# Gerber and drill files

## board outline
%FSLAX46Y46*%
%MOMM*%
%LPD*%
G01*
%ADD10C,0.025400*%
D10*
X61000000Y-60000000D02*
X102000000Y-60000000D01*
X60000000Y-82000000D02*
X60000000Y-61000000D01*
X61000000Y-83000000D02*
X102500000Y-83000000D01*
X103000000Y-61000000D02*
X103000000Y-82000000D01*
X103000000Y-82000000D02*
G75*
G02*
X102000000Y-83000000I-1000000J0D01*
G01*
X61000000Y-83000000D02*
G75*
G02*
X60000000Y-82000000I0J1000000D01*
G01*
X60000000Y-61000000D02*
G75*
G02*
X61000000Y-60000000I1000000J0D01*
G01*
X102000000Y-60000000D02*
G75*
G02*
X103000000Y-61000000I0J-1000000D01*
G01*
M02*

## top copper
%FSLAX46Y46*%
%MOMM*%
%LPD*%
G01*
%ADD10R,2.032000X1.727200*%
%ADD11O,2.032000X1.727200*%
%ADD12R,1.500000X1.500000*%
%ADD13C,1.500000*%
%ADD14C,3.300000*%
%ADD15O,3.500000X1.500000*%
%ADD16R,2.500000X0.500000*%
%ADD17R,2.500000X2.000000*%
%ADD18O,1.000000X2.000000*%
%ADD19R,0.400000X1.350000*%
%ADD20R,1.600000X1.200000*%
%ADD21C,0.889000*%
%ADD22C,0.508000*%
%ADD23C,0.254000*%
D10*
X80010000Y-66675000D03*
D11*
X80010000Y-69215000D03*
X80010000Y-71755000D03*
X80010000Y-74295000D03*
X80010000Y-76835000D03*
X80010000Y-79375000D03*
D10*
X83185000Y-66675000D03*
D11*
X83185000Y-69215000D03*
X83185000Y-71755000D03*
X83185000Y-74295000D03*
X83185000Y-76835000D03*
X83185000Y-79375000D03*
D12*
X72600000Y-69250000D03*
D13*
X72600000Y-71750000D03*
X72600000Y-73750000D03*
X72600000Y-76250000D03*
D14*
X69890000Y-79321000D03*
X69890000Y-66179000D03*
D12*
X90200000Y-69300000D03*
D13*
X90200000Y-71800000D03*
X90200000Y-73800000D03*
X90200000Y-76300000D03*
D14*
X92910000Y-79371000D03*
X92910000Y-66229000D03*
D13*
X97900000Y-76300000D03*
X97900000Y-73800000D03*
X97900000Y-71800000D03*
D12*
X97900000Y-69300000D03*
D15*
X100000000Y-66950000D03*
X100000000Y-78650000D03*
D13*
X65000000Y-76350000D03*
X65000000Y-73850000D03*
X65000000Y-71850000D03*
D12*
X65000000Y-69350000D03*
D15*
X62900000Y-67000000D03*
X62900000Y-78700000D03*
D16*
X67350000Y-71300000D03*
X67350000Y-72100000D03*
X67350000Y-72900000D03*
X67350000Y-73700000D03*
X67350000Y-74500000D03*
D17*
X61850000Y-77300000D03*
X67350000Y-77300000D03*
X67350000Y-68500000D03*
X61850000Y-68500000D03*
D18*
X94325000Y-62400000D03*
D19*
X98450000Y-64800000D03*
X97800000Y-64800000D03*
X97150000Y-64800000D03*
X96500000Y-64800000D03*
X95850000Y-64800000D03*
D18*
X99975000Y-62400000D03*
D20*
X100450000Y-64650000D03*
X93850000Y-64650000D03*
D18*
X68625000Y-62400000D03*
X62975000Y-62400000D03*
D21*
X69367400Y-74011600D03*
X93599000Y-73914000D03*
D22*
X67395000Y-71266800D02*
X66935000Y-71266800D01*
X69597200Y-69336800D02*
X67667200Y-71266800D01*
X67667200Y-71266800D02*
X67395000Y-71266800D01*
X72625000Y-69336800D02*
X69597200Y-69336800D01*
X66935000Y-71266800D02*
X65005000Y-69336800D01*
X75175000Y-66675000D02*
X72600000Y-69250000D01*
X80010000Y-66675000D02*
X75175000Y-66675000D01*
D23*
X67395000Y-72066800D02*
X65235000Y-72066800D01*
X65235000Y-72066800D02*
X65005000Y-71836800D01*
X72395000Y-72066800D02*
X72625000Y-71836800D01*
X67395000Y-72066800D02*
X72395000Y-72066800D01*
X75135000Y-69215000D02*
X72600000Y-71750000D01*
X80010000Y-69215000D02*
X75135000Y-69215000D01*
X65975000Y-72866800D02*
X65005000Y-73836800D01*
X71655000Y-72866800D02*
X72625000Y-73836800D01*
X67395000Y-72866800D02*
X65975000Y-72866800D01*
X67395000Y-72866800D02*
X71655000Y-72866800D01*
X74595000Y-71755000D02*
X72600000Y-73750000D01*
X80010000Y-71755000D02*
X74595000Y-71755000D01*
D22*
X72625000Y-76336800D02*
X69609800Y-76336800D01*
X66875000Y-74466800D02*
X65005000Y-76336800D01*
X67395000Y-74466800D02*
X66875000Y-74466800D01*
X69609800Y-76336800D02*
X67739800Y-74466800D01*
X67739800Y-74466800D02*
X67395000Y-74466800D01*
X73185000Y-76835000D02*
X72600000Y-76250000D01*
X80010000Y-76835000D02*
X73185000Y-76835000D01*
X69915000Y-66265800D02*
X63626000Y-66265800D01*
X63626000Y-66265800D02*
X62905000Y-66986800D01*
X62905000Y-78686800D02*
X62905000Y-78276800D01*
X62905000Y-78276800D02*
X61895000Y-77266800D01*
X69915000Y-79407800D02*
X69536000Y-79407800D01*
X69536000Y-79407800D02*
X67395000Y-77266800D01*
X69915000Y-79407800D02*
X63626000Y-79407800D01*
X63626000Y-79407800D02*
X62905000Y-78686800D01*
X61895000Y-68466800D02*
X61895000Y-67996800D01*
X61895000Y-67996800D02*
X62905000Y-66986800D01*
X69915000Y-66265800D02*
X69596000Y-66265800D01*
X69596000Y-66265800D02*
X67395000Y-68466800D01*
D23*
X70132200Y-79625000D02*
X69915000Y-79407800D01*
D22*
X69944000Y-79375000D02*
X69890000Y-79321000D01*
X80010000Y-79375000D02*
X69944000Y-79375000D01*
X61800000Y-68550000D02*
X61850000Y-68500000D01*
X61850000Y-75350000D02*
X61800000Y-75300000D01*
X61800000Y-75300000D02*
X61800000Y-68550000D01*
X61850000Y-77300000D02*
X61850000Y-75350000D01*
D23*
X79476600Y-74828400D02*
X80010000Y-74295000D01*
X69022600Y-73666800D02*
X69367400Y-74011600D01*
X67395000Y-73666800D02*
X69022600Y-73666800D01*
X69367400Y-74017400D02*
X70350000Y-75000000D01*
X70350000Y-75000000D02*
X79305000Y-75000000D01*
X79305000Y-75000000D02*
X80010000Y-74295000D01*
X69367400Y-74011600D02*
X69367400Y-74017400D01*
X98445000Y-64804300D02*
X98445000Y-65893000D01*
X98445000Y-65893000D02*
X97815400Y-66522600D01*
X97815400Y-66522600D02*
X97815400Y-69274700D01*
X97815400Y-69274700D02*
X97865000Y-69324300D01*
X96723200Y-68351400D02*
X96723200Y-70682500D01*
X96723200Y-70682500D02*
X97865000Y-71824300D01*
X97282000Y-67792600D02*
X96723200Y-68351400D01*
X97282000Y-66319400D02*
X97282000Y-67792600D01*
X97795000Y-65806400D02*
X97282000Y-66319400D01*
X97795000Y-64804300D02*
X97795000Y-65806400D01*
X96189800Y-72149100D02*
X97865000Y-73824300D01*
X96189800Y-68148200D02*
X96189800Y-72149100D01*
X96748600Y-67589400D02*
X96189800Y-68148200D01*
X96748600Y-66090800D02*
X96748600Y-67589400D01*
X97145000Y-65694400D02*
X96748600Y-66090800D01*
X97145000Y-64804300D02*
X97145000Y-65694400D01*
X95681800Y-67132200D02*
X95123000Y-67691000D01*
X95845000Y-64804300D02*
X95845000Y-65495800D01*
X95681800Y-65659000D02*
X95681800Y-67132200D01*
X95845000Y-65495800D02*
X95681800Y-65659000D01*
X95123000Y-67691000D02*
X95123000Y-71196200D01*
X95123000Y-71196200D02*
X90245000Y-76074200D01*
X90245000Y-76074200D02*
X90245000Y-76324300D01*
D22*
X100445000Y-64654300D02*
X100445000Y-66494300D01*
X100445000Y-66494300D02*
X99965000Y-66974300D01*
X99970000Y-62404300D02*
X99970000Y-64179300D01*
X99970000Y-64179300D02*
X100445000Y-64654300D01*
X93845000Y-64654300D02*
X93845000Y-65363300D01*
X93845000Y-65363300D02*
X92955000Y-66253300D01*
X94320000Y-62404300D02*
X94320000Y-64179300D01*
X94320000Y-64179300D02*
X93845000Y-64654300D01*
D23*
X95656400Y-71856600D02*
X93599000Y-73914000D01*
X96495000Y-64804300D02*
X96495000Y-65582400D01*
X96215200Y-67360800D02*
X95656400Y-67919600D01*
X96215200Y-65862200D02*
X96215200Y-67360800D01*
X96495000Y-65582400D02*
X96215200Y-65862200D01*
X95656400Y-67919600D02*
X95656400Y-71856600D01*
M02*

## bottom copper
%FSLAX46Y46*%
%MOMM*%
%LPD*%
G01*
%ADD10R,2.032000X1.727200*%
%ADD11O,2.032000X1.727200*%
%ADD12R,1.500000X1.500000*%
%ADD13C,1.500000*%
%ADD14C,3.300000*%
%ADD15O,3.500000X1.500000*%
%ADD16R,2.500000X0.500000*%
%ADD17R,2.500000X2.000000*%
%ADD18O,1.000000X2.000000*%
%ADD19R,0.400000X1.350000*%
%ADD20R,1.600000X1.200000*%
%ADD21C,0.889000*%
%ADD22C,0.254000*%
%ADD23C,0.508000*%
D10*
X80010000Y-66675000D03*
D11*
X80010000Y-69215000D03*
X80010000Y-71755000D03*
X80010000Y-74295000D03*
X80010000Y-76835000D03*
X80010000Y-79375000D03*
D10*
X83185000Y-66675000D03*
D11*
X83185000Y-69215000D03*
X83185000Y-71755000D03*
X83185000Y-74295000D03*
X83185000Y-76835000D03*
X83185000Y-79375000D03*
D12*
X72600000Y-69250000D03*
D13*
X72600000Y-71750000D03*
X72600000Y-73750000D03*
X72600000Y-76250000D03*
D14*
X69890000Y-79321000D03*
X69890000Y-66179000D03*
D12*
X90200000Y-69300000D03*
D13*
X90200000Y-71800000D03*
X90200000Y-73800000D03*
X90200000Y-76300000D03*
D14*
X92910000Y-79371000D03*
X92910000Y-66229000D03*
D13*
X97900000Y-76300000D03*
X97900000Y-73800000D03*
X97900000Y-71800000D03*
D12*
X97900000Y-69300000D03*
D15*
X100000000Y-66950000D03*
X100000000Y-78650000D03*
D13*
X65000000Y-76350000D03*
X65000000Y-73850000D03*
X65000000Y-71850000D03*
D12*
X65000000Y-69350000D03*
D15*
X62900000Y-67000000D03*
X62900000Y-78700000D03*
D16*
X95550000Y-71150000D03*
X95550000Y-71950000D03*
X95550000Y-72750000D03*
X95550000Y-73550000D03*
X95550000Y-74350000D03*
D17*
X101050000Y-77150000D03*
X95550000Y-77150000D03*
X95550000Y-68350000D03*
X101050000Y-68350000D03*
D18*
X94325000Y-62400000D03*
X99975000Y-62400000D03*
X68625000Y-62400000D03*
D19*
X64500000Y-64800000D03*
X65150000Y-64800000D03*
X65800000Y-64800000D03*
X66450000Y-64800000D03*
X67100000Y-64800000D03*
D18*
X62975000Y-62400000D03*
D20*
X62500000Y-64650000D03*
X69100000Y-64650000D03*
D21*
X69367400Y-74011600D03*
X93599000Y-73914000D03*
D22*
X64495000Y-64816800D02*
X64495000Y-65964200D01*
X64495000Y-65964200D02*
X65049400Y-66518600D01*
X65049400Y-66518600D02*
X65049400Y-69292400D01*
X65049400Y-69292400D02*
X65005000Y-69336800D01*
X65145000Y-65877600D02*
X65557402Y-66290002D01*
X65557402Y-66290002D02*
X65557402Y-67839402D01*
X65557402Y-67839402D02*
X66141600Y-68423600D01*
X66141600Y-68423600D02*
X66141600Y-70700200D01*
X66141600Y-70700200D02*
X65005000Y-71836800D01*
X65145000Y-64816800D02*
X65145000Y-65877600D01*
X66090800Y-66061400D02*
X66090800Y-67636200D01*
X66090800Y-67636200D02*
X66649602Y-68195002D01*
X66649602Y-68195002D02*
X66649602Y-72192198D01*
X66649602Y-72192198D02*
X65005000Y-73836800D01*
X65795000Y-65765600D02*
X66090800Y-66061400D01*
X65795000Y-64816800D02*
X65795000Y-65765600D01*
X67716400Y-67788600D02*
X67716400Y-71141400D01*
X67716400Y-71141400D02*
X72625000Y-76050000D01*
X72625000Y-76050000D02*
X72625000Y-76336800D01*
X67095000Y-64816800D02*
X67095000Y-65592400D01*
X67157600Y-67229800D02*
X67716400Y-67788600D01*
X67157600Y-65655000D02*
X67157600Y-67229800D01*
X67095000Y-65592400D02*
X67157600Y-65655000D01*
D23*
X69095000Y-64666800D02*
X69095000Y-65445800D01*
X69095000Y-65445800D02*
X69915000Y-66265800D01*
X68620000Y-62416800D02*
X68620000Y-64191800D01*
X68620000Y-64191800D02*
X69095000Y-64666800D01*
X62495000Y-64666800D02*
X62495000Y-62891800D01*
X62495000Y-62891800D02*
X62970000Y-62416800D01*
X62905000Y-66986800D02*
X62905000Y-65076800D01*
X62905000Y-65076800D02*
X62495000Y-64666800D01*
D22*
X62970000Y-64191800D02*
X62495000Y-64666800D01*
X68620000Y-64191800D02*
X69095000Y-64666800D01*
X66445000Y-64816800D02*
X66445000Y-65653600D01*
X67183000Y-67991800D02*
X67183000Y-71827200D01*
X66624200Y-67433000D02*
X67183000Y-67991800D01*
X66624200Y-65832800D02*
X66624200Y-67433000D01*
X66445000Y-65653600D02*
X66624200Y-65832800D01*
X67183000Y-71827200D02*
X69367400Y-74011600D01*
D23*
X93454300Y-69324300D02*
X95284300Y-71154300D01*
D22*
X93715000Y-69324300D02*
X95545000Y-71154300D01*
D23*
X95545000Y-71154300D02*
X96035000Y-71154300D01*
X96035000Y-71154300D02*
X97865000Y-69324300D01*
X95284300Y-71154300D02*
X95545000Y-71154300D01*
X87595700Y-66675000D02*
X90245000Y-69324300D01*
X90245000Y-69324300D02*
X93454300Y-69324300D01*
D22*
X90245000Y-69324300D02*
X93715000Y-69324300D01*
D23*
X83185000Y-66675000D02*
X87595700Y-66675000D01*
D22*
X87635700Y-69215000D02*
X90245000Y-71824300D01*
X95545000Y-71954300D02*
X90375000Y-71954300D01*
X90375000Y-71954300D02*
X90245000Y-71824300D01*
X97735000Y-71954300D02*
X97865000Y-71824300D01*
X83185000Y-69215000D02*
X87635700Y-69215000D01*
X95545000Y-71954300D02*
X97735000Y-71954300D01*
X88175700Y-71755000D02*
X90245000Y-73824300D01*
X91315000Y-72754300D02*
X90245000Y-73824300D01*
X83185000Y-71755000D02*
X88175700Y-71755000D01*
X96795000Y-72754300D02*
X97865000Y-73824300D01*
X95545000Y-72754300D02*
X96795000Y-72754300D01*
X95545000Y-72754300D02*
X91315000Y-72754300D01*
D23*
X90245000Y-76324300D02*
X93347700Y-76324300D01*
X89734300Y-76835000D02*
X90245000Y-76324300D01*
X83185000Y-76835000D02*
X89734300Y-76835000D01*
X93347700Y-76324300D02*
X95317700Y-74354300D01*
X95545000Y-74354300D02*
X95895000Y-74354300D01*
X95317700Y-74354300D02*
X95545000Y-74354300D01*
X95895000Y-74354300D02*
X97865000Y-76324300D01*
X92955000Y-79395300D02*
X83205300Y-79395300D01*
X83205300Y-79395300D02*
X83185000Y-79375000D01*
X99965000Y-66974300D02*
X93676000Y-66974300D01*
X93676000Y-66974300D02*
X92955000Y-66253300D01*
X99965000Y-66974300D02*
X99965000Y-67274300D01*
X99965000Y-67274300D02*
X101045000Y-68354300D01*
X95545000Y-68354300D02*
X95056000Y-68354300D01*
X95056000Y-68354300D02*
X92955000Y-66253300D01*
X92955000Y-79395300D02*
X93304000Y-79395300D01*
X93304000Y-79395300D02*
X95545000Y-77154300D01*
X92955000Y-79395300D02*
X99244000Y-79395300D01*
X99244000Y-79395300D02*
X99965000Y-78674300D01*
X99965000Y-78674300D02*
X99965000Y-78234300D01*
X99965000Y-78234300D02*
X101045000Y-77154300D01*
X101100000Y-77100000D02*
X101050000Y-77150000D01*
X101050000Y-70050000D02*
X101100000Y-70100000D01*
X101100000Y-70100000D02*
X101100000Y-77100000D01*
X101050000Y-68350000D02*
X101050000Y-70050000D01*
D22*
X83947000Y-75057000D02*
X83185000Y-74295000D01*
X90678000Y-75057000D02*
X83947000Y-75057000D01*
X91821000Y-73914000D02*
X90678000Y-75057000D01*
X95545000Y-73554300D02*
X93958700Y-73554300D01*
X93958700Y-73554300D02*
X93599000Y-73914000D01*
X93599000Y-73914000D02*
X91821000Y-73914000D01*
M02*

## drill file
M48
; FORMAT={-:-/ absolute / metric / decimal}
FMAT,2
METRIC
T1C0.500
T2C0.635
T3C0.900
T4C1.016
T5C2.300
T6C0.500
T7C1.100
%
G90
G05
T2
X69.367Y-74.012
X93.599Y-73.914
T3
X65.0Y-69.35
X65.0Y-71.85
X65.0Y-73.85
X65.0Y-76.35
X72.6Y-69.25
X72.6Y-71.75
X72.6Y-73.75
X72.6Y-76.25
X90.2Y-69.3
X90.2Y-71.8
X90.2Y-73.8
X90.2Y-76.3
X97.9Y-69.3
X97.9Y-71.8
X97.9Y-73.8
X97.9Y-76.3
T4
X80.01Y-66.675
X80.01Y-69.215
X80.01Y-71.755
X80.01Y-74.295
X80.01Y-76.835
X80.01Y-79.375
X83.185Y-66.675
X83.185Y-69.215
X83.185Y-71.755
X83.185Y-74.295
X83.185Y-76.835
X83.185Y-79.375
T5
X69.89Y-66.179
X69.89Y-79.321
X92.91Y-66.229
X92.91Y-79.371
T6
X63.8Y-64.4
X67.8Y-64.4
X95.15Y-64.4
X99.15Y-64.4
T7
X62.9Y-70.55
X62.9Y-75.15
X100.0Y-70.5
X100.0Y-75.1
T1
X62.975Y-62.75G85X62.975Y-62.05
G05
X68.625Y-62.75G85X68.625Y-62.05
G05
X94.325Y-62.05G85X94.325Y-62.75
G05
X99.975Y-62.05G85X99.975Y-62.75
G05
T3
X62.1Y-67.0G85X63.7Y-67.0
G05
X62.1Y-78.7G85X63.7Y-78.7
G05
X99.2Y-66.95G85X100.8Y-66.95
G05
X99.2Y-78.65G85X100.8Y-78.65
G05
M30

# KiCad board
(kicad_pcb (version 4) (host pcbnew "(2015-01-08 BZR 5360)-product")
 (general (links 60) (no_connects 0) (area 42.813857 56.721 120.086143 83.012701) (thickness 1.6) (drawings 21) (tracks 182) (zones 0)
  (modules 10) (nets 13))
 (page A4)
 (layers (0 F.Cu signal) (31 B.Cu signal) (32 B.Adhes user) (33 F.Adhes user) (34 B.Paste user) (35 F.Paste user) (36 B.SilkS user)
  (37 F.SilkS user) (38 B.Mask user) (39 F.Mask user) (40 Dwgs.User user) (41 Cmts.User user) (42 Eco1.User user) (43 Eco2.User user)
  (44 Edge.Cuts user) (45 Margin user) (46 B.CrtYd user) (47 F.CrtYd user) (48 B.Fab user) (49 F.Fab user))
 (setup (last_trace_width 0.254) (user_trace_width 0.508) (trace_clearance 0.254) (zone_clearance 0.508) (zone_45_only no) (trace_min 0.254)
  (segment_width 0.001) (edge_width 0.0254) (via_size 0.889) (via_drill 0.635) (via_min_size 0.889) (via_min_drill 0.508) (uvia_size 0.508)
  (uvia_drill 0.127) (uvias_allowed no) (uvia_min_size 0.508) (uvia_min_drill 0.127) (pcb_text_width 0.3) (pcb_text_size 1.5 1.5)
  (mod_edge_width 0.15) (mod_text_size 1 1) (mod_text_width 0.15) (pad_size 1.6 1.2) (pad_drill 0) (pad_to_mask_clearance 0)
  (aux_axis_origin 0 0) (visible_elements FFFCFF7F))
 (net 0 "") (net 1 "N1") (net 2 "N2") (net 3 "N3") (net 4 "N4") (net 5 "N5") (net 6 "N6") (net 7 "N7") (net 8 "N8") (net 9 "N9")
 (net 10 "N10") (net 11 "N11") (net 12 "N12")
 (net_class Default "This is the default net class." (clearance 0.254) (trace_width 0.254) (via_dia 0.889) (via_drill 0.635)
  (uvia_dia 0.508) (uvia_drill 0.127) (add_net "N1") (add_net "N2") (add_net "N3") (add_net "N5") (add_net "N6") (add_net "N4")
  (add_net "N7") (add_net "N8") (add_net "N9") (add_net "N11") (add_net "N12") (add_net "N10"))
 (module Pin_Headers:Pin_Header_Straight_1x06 (layer F.Cu) (at 80.01 73.025 270)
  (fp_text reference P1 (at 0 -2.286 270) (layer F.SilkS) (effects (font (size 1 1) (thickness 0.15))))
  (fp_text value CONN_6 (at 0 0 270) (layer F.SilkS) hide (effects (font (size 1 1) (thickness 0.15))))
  (pad 1 thru_hole rect (at -6.35 0 270) (size 1.7272 2.032) (drill 1.016) (layers *.Cu *.Mask F.SilkS) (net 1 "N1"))
  (pad 2 thru_hole oval (at -3.81 0 270) (size 1.7272 2.032) (drill 1.016) (layers *.Cu *.Mask F.SilkS) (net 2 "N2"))
  (pad 3 thru_hole oval (at -1.27 0 270) (size 1.7272 2.032) (drill 1.016) (layers *.Cu *.Mask F.SilkS) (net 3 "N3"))
  (pad 4 thru_hole oval (at 1.27 0 270) (size 1.7272 2.032) (drill 1.016) (layers *.Cu *.Mask F.SilkS) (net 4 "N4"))
  (pad 5 thru_hole oval (at 3.81 0 270) (size 1.7272 2.032) (drill 1.016) (layers *.Cu *.Mask F.SilkS) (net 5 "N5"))
  (pad 6 thru_hole oval (at 6.35 0 270) (size 1.7272 2.032) (drill 1.016) (layers *.Cu *.Mask F.SilkS) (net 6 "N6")))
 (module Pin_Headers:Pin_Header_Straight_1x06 (layer F.Cu) (at 83.185 73.025 270)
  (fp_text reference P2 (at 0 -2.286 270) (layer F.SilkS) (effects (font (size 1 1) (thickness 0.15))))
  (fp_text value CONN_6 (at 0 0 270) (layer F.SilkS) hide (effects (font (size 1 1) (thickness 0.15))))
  (pad 1 thru_hole rect (at -6.35 0 270) (size 1.7272 2.032) (drill 1.016) (layers *.Cu *.Mask F.SilkS) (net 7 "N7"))
  (pad 2 thru_hole oval (at -3.81 0 270) (size 1.7272 2.032) (drill 1.016) (layers *.Cu *.Mask F.SilkS) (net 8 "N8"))
  (pad 3 thru_hole oval (at -1.27 0 270) (size 1.7272 2.032) (drill 1.016) (layers *.Cu *.Mask F.SilkS) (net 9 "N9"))
  (pad 4 thru_hole oval (at 1.27 0 270) (size 1.7272 2.032) (drill 1.016) (layers *.Cu *.Mask F.SilkS) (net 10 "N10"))
  (pad 5 thru_hole oval (at 3.81 0 270) (size 1.7272 2.032) (drill 1.016) (layers *.Cu *.Mask F.SilkS) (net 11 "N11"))
  (pad 6 thru_hole oval (at 6.35 0 270) (size 1.7272 2.032) (drill 1.016) (layers *.Cu *.Mask F.SilkS) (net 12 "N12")))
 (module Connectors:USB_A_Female (layer F.Cu) (at 72.6 69.25 270)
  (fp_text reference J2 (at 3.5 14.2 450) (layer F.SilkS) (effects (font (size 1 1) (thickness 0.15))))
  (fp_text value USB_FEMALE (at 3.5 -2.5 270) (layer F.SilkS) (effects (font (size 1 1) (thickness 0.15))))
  (pad 1 thru_hole rect (at 0 0 270) (size 1.5 1.5) (drill 0.9) (layers *.Cu *.Mask F.SilkS) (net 1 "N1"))
  (pad 2 thru_hole circle (at 2.5 0 270) (size 1.5 1.5) (drill 0.9) (layers *.Cu *.Mask F.SilkS) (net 2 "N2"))
  (pad 3 thru_hole circle (at 4.5 0 270) (size 1.5 1.5) (drill 0.9) (layers *.Cu *.Mask F.SilkS) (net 3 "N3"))
  (pad 4 thru_hole circle (at 7 0 270) (size 1.5 1.5) (drill 0.9) (layers *.Cu *.Mask F.SilkS) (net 5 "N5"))
  (pad 5 thru_hole circle (at 10.071 2.71 270) (size 3.3 3.3) (drill 2.3) (layers *.Cu *.Mask F.SilkS) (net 6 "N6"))
  (pad 5 thru_hole circle (at -3.071 2.71 270) (size 3.3 3.3) (drill 2.3) (layers *.Cu *.Mask F.SilkS) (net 6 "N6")))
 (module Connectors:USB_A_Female (layer B.Cu) (at 90.2 69.3 270)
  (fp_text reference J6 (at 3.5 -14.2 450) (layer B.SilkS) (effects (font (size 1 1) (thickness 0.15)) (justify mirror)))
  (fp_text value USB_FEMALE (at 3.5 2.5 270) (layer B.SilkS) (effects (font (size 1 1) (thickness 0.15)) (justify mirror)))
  (pad 1 thru_hole rect (at 0 0 270) (size 1.5 1.5) (drill 0.9) (layers *.Cu *.Mask B.SilkS) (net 7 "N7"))
  (pad 2 thru_hole circle (at 2.5 0 270) (size 1.5 1.5) (drill 0.9) (layers *.Cu *.Mask B.SilkS) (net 8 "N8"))
  (pad 3 thru_hole circle (at 4.5 0 270) (size 1.5 1.5) (drill 0.9) (layers *.Cu *.Mask B.SilkS) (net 9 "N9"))
  (pad 4 thru_hole circle (at 7 0 270) (size 1.5 1.5) (drill 0.9) (layers *.Cu *.Mask B.SilkS) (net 11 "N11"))
  (pad 5 thru_hole circle (at 10.071 -2.71 270) (size 3.3 3.3) (drill 2.3) (layers *.Cu *.Mask B.SilkS) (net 12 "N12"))
  (pad 5 thru_hole circle (at -3.071 -2.71 270) (size 3.3 3.3) (drill 2.3) (layers *.Cu *.Mask B.SilkS) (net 12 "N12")))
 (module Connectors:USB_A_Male (layer F.Cu) (at 97.9 69.3 270)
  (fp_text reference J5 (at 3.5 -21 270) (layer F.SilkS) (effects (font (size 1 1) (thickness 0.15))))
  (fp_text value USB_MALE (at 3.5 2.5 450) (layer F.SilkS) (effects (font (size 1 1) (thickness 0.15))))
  (pad 4 thru_hole circle (at 7 0 90) (size 1.5 1.5) (drill 0.9) (layers *.Cu *.Mask F.SilkS) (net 11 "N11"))
  (pad 3 thru_hole circle (at 4.5 0 90) (size 1.5 1.5) (drill 0.9) (layers *.Cu *.Mask F.SilkS) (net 9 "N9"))
  (pad 2 thru_hole circle (at 2.5 0 90) (size 1.5 1.5) (drill 0.9) (layers *.Cu *.Mask F.SilkS) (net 8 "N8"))
  (pad 1 thru_hole rect (at 0 0 90) (size 1.5 1.5) (drill 0.9) (layers *.Cu *.Mask F.SilkS) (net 7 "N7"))
  (pad 5 thru_hole oval (at -2.35 -2.1 90) (size 1.5 3.5) (drill oval 0.9 2.5) (layers *.Cu *.Mask F.SilkS) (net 12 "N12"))
  (pad 5 thru_hole oval (at 9.35 -2.1 90) (size 1.5 3.5) (drill oval 0.9 2.5) (layers *.Cu *.Mask F.SilkS) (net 12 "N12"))
  (pad "" np_thru_hole circle (at 5.8 -2.1 90) (size 1.1 1.1) (drill 1.1) (layers *.Cu *.Mask F.SilkS))
  (pad "" np_thru_hole circle (at 1.2 -2.1 90) (size 1.1 1.1) (drill 1.1) (layers *.Cu *.Mask F.SilkS)))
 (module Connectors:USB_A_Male (layer B.Cu) (at 65 69.35 270)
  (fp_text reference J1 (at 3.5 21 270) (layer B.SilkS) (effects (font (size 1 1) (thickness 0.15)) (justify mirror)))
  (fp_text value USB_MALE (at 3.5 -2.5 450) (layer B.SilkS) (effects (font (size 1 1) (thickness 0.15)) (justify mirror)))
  (pad 4 thru_hole circle (at 7 0 90) (size 1.5 1.5) (drill 0.9) (layers *.Cu *.Mask B.SilkS) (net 5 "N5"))
  (pad 3 thru_hole circle (at 4.5 0 90) (size 1.5 1.5) (drill 0.9) (layers *.Cu *.Mask B.SilkS) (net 3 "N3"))
  (pad 2 thru_hole circle (at 2.5 0 90) (size 1.5 1.5) (drill 0.9) (layers *.Cu *.Mask B.SilkS) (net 2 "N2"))
  (pad 1 thru_hole rect (at 0 0 90) (size 1.5 1.5) (drill 0.9) (layers *.Cu *.Mask B.SilkS) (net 1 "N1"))
  (pad 5 thru_hole oval (at -2.35 2.1 90) (size 1.5 3.5) (drill oval 0.9 2.5) (layers *.Cu *.Mask B.SilkS) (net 6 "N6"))
  (pad 5 thru_hole oval (at 9.35 2.1 90) (size 1.5 3.5) (drill oval 0.9 2.5) (layers *.Cu *.Mask B.SilkS) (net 6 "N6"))
  (pad "" np_thru_hole circle (at 5.8 2.1 90) (size 1.1 1.1) (drill 1.1) (layers *.Cu *.Mask B.SilkS))
  (pad "" np_thru_hole circle (at 1.2 2.1 90) (size 1.1 1.1) (drill 1.1) (layers *.Cu *.Mask B.SilkS)))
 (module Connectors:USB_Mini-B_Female (layer F.Cu) (at 67.35 71.3 270)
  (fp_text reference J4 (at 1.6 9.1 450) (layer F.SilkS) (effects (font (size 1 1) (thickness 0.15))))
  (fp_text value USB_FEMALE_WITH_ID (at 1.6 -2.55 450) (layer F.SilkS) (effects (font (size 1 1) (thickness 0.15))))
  (pad 1 smd rect (at 0 0 90) (size 0.5 2.5) (layers F.Cu F.Paste F.Mask) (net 1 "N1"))
  (pad 2 smd rect (at 0.8 0 90) (size 0.5 2.5) (layers F.Cu F.Paste F.Mask) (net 2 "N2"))
  (pad 3 smd rect (at 1.6 0 90) (size 0.5 2.5) (layers F.Cu F.Paste F.Mask) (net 3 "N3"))
  (pad 4 smd rect (at 2.4 0 90) (size 0.5 2.5) (layers F.Cu F.Paste F.Mask) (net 4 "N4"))
  (pad 5 smd rect (at 3.2 0 90) (size 0.5 2.5) (layers F.Cu F.Paste F.Mask) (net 5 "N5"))
  (pad 6 smd rect (at 6 5.5 90) (size 2 2.5) (layers F.Cu F.Paste F.Mask) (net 6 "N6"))
  (pad 6 smd rect (at 6 0 90) (size 2 2.5) (layers F.Cu F.Paste F.Mask) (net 6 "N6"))
  (pad 6 smd rect (at -2.8 0 90) (size 2 2.5) (layers F.Cu F.Paste F.Mask) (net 6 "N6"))
  (pad 6 smd rect (at -2.8 5.5 90) (size 2 2.5) (layers F.Cu F.Paste F.Mask) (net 6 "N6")))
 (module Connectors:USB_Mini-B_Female (layer B.Cu) (at 95.55 71.15 270)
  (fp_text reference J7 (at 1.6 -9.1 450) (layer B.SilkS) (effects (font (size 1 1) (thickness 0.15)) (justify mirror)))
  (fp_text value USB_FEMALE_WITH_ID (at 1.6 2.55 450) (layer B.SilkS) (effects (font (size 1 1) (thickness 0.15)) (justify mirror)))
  (pad 1 smd rect (at 0 0 90) (size 0.5 2.5) (layers B.Cu B.Paste B.Mask) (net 7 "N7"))
  (pad 2 smd rect (at 0.8 0 90) (size 0.5 2.5) (layers B.Cu B.Paste B.Mask) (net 8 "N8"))
  (pad 3 smd rect (at 1.6 0 90) (size 0.5 2.5) (layers B.Cu B.Paste B.Mask) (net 9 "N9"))
  (pad 4 smd rect (at 2.4 0 90) (size 0.5 2.5) (layers B.Cu B.Paste B.Mask) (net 10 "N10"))
  (pad 5 smd rect (at 3.2 0 90) (size 0.5 2.5) (layers B.Cu B.Paste B.Mask) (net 11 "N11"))
  (pad 6 smd rect (at 6 -5.5 90) (size 2 2.5) (layers B.Cu B.Paste B.Mask) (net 12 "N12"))
  (pad 6 smd rect (at 6 0 90) (size 2 2.5) (layers B.Cu B.Paste B.Mask) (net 12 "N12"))
  (pad 6 smd rect (at -2.8 0 90) (size 2 2.5) (layers B.Cu B.Paste B.Mask) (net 12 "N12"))
  (pad 6 smd rect (at -2.8 -5.5 90) (size 2 2.5) (layers B.Cu B.Paste B.Mask) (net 12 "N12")))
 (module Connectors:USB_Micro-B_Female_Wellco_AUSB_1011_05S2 (layer F.Cu) (at 98.45 64.8 180)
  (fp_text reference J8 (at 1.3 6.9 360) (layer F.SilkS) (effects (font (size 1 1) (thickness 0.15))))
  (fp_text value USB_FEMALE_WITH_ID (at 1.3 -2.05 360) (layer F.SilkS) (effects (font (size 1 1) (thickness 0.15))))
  (pad 6 thru_hole oval (at 4.125 2.4) (size 1 2) (drill oval 0.5 1.2) (layers *.Cu *.Mask F.SilkS) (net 12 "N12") (clearance 0.25))
  (pad 1 smd rect (at 0 0) (size 0.4 1.35) (layers F.Cu F.Paste F.Mask) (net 7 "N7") (clearance 0.24999))
  (pad 2 smd rect (at 0.65 0) (size 0.4 1.35) (layers F.Cu F.Paste F.Mask) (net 8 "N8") (clearance 0.25))
  (pad 3 smd rect (at 1.3 0) (size 0.4 1.35) (layers F.Cu F.Paste F.Mask) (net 9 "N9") (clearance 0.25))
  (pad 4 smd rect (at 1.95 0) (size 0.4 1.35) (layers F.Cu F.Paste F.Mask) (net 10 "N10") (clearance 0.25))
  (pad 5 smd rect (at 2.6 0) (size 0.4 1.35) (layers F.Cu F.Paste F.Mask) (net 11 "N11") (clearance 0.24999))
  (pad 6 thru_hole oval (at -1.525 2.4) (size 1 2) (drill oval 0.5 1.2) (layers *.Cu *.Mask F.SilkS) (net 12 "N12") (clearance 0.25))
  (pad "" np_thru_hole circle (at 3.3 0.4) (size 0.5 0.5) (drill 0.5) (layers *.Cu *.Mask F.SilkS) (clearance 0.24999))
  (pad "" np_thru_hole circle (at -0.7 0.4) (size 0.5 0.5) (drill 0.5) (layers *.Cu *.Mask F.SilkS) (clearance 0.249999))
  (pad 6 smd rect (at -2 0.15) (size 1.6 1.2) (layers F.Cu F.Paste F.Mask) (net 12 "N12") (clearance 0.249999))
  (pad 6 smd rect (at 4.6 0.15) (size 1.6 1.2) (layers F.Cu F.Paste F.Mask) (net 12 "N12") (clearance 0.24999)))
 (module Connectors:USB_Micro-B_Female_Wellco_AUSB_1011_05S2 (layer B.Cu) (at 64.5 64.8)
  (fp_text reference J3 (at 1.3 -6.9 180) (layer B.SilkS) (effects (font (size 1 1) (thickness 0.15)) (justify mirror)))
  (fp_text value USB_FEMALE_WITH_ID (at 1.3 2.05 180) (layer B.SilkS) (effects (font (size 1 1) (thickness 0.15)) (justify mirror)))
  (pad 6 thru_hole oval (at 4.125 -2.4 180) (size 1 2) (drill oval 0.5 1.2) (layers *.Cu *.Mask B.SilkS) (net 6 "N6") (clearance 0.25))
  (pad 1 smd rect (at 0 0 180) (size 0.4 1.35) (layers B.Cu B.Paste B.Mask) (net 1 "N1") (clearance 0.24999))
  (pad 2 smd rect (at 0.65 0 180) (size 0.4 1.35) (layers B.Cu B.Paste B.Mask) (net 2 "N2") (clearance 0.25))
  (pad 3 smd rect (at 1.3 0 180) (size 0.4 1.35) (layers B.Cu B.Paste B.Mask) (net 3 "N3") (clearance 0.25))
  (pad 4 smd rect (at 1.95 0 180) (size 0.4 1.35) (layers B.Cu B.Paste B.Mask) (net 4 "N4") (clearance 0.25))
  (pad 5 smd rect (at 2.6 0 180) (size 0.4 1.35) (layers B.Cu B.Paste B.Mask) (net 5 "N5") (clearance 0.24999))
  (pad 6 thru_hole oval (at -1.525 -2.4 180) (size 1 2) (drill oval 0.5 1.2) (layers *.Cu *.Mask B.SilkS) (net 6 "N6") (clearance 0.25))
  (pad "" np_thru_hole circle (at 3.3 -0.4 180) (size 0.5 0.5) (drill 0.5) (layers *.Cu *.Mask B.SilkS) (clearance 0.24999))
  (pad "" np_thru_hole circle (at -0.7 -0.4 180) (size 0.5 0.5) (drill 0.5) (layers *.Cu *.Mask B.SilkS) (clearance 0.249999))
  (pad 6 smd rect (at -2 -0.15 180) (size 1.6 1.2) (layers B.Cu B.Paste B.Mask) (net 6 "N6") (clearance 0.249999))
  (pad 6 smd rect (at 4.6 -0.15 180) (size 1.6 1.2) (layers B.Cu B.Paste B.Mask) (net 6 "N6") (clearance 0.24999)))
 (gr_line (start 61 60) (end 102 60) (angle 90) (layer Edge.Cuts) (width 0.0254))
 (gr_line (start 60 82) (end 60 61) (angle 90) (layer Edge.Cuts) (width 0.0254))
 (gr_line (start 61 83) (end 102.5 83) (angle 90) (layer Edge.Cuts) (width 0.0254))
 (gr_line (start 103 61) (end 103 82) (angle 90) (layer Edge.Cuts) (width 0.0254))
 (gr_arc (start 102 82) (end 103 82) (angle 90) (layer Edge.Cuts) (width 0.0254))
 (gr_arc (start 61 82) (end 61 83) (angle 90) (layer Edge.Cuts) (width 0.0254))
 (gr_arc (start 61 61) (end 60 61) (angle 90) (layer Edge.Cuts) (width 0.0254))
 (gr_arc (start 102 61) (end 102 60) (angle 90) (layer Edge.Cuts) (width 0.0254))
 (segment (start 67.395 71.2668) (end 66.935 71.2668) (width 0.508) (layer F.Cu) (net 1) (status 30))
 (segment (start 69.5972 69.3368) (end 67.6672 71.2668) (width 0.508) (layer F.Cu) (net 1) (status 20))
 (segment (start 67.6672 71.2668) (end 67.395 71.2668) (width 0.508) (layer F.Cu) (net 1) (status 30))
 (segment (start 64.495 64.8168) (end 64.495 65.9642) (width 0.254) (layer B.Cu) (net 1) (status 10))
 (segment (start 64.495 65.9642) (end 65.0494 66.5186) (width 0.254) (layer B.Cu) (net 1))
 (segment (start 72.625 69.3368) (end 69.5972 69.3368) (width 0.508) (layer F.Cu) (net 1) (status 10))
 (segment (start 66.935 71.2668) (end 65.005 69.3368) (width 0.508) (layer F.Cu) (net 1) (status 30))
 (segment (start 65.0494 66.5186) (end 65.0494 69.2924) (width 0.254) (layer B.Cu) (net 1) (status 20))
 (segment (start 65.0494 69.2924) (end 65.005 69.3368) (width 0.254) (layer B.Cu) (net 1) (status 30))
 (segment (start 75.175 66.675) (end 72.6 69.25) (width 0.508) (layer F.Cu) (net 1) (status 20))
 (segment (start 80.01 66.675) (end 75.175 66.675) (width 0.508) (layer F.Cu) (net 1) (status 10))
 (segment (start 67.395 72.0668) (end 65.235 72.0668) (width 0.254) (layer F.Cu) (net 2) (status 30))
 (segment (start 65.235 72.0668) (end 65.005 71.8368) (width 0.254) (layer F.Cu) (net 2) (status 30))
 (segment (start 65.145 65.8776) (end 65.557402 66.290002) (width 0.254) (layer B.Cu) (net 2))
 (segment (start 72.395 72.0668) (end 72.625 71.8368) (width 0.254) (layer F.Cu) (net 2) (status 30))
 (segment (start 65.557402 66.290002) (end 65.557402 67.839402) (width 0.254) (layer B.Cu) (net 2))
 (segment (start 65.557402 67.839402) (end 66.1416 68.4236) (width 0.254) (layer B.Cu) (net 2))
 (segment (start 66.1416 68.4236) (end 66.1416 70.7002) (width 0.254) (layer B.Cu) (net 2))
 (segment (start 66.1416 70.7002) (end 65.005 71.8368) (width 0.254) (layer B.Cu) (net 2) (status 20))
 (segment (start 65.145 64.8168) (end 65.145 65.8776) (width 0.254) (layer B.Cu) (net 2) (status 10))
 (segment (start 67.395 72.0668) (end 72.395 72.0668) (width 0.254) (layer F.Cu) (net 2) (status 30))
 (segment (start 75.135 69.215) (end 72.6 71.75) (width 0.254) (layer F.Cu) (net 2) (status 20))
 (segment (start 80.01 69.215) (end 75.135 69.215) (width 0.254) (layer F.Cu) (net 2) (status 10))
 (segment (start 65.975 72.8668) (end 65.005 73.8368) (width 0.254) (layer F.Cu) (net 3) (status 20))
 (segment (start 71.655 72.8668) (end 72.625 73.8368) (width 0.254) (layer F.Cu) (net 3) (status 20))
 (segment (start 66.0908 66.0614) (end 66.0908 67.6362) (width 0.254) (layer B.Cu) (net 3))
 (segment (start 66.0908 67.6362) (end 66.649602 68.195002) (width 0.254) (layer B.Cu) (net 3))
 (segment (start 66.649602 68.195002) (end 66.649602 72.192198) (width 0.254) (layer B.Cu) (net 3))
 (segment (start 66.649602 72.192198) (end 65.005 73.8368) (width 0.254) (layer B.Cu) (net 3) (status 20))
 (segment (start 65.795 65.7656) (end 66.0908 66.0614) (width 0.254) (layer B.Cu) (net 3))
 (segment (start 65.795 64.8168) (end 65.795 65.7656) (width 0.254) (layer B.Cu) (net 3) (status 10))
 (segment (start 67.395 72.8668) (end 65.975 72.8668) (width 0.254) (layer F.Cu) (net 3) (status 10))
 (segment (start 67.395 72.8668) (end 71.655 72.8668) (width 0.254) (layer F.Cu) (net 3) (status 10))
 (segment (start 74.595 71.755) (end 72.6 73.75) (width 0.254) (layer F.Cu) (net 3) (status 20))
 (segment (start 80.01 71.755) (end 74.595 71.755) (width 0.254) (layer F.Cu) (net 3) (status 10))
 (segment (start 67.7164 67.7886) (end 67.7164 71.1414) (width 0.254) (layer B.Cu) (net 5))
 (segment (start 72.625 76.3368) (end 69.6098 76.3368) (width 0.508) (layer F.Cu) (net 5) (status 10))
 (segment (start 67.7164 71.1414) (end 72.625 76.05) (width 0.254) (layer B.Cu) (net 5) (status 20))
 (segment (start 72.625 76.05) (end 72.625 76.3368) (width 0.254) (layer B.Cu) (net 5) (status 30))
 (segment (start 66.875 74.4668) (end 65.005 76.3368) (width 0.508) (layer F.Cu) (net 5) (status 30))
 (segment (start 67.095 64.8168) (end 67.095 65.5924) (width 0.254) (layer B.Cu) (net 5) (status 10))
 (segment (start 67.1576 67.2298) (end 67.7164 67.7886) (width 0.254) (layer B.Cu) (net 5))
 (segment (start 67.1576 65.655) (end 67.1576 67.2298) (width 0.254) (layer B.Cu) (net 5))
 (segment (start 67.095 65.5924) (end 67.1576 65.655) (width 0.254) (layer B.Cu) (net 5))
 (segment (start 67.395 74.4668) (end 66.875 74.4668) (width 0.508) (layer F.Cu) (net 5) (status 30))
 (segment (start 69.6098 76.3368) (end 67.7398 74.4668) (width 0.508) (layer F.Cu) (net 5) (status 20))
 (segment (start 67.7398 74.4668) (end 67.395 74.4668) (width 0.508) (layer F.Cu) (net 5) (status 30))
 (segment (start 73.185 76.835) (end 72.6 76.25) (width 0.508) (layer F.Cu) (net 5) (status 20))
 (segment (start 80.01 76.835) (end 73.185 76.835) (width 0.508) (layer F.Cu) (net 5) (status 10))
 (segment (start 69.915 66.2658) (end 63.626 66.2658) (width 0.508) (layer F.Cu) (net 6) (status 30))
 (segment (start 63.626 66.2658) (end 62.905 66.9868) (width 0.508) (layer F.Cu) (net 6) (status 30))
 (segment (start 69.095 64.6668) (end 69.095 65.4458) (width 0.508) (layer B.Cu) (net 6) (status 30))
 (segment (start 69.095 65.4458) (end 69.915 66.2658) (width 0.508) (layer B.Cu) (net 6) (status 30))
 (segment (start 68.62 62.4168) (end 68.62 64.1918) (width 0.508) (layer B.Cu) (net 6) (status 30))
 (segment (start 68.62 64.1918) (end 69.095 64.6668) (width 0.508) (layer B.Cu) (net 6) (status 30))
 (segment (start 62.495 64.6668) (end 62.495 62.8918) (width 0.508) (layer B.Cu) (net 6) (status 30))
 (segment (start 62.495 62.8918) (end 62.97 62.4168) (width 0.508) (layer B.Cu) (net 6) (status 30))
 (segment (start 62.905 66.9868) (end 62.905 65.0768) (width 0.508) (layer B.Cu) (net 6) (status 30))
 (segment (start 62.905 65.0768) (end 62.495 64.6668) (width 0.508) (layer B.Cu) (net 6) (status 30))
 (segment (start 62.905 78.6868) (end 62.905 78.2768) (width 0.508) (layer F.Cu) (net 6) (status 30))
 (segment (start 62.905 78.2768) (end 61.895 77.2668) (width 0.508) (layer F.Cu) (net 6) (status 30))
 (segment (start 69.915 79.4078) (end 69.536 79.4078) (width 0.508) (layer F.Cu) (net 6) (status 30))
 (segment (start 69.536 79.4078) (end 67.395 77.2668) (width 0.508) (layer F.Cu) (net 6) (status 30))
 (segment (start 69.915 79.4078) (end 63.626 79.4078) (width 0.508) (layer F.Cu) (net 6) (status 30))
 (segment (start 63.626 79.4078) (end 62.905 78.6868) (width 0.508) (layer F.Cu) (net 6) (status 30))
 (segment (start 61.895 68.4668) (end 61.895 67.9968) (width 0.508) (layer F.Cu) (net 6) (status 30))
 (segment (start 61.895 67.9968) (end 62.905 66.9868) (width 0.508) (layer F.Cu) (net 6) (status 30))
 (segment (start 69.915 66.2658) (end 69.596 66.2658) (width 0.508) (layer F.Cu) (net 6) (status 30))
 (segment (start 69.596 66.2658) (end 67.395 68.4668) (width 0.508) (layer F.Cu) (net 6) (status 30))
 (segment (start 62.97 64.1918) (end 62.495 64.6668) (width 0.254) (layer B.Cu) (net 6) (status 30))
 (segment (start 68.62 64.1918) (end 69.095 64.6668) (width 0.254) (layer B.Cu) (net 6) (status 30))
 (segment (start 70.1322 79.625) (end 69.915 79.4078) (width 0.254) (layer F.Cu) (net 6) (status 30))
 (segment (start 69.944 79.375) (end 69.89 79.321) (width 0.508) (layer F.Cu) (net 6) (status 30))
 (segment (start 80.01 79.375) (end 69.944 79.375) (width 0.508) (layer F.Cu) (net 6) (status 30))
 (segment (start 61.8 68.55) (end 61.85 68.5) (width 0.508) (layer F.Cu) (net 6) (status 30))
 (segment (start 61.85 75.35) (end 61.8 75.3) (width 0.508) (layer F.Cu) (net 6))
 (segment (start 61.8 75.3) (end 61.8 68.55) (width 0.508) (layer F.Cu) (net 6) (status 20))
 (segment (start 61.85 77.3) (end 61.85 75.35) (width 0.508) (layer F.Cu) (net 6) (status 10))
 (segment (start 79.4766 74.8284) (end 80.01 74.295) (width 0.254) (layer F.Cu) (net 4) (status 30))
 (segment (start 66.445 64.8168) (end 66.445 65.6536) (width 0.254) (layer B.Cu) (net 4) (status 10))
 (segment (start 67.183 67.9918) (end 67.183 71.8272) (width 0.254) (layer B.Cu) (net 4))
 (segment (start 66.6242 67.433) (end 67.183 67.9918) (width 0.254) (layer B.Cu) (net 4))
 (segment (start 66.6242 65.8328) (end 66.6242 67.433) (width 0.254) (layer B.Cu) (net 4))
 (segment (start 66.445 65.6536) (end 66.6242 65.8328) (width 0.254) (layer B.Cu) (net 4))
 (segment (start 67.183 71.8272) (end 69.3674 74.0116) (width 0.254) (layer B.Cu) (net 4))
 (segment (start 69.0226 73.6668) (end 69.3674 74.0116) (width 0.254) (layer F.Cu) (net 4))
 (via (at 69.3674 74.0116) (size 0.889) (layers F.Cu B.Cu) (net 4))
 (segment (start 67.395 73.6668) (end 69.0226 73.6668) (width 0.254) (layer F.Cu) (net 4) (status 10))
 (segment (start 69.3674 74.0174) (end 70.35 75) (width 0.254) (layer F.Cu) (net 4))
 (segment (start 70.35 75) (end 79.305 75) (width 0.254) (layer F.Cu) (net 4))
 (segment (start 79.305 75) (end 80.01 74.295) (width 0.254) (layer F.Cu) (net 4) (status 20))
 (segment (start 69.3674 74.0116) (end 69.3674 74.0174) (width 0.254) (layer F.Cu) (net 4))
 (segment (start 93.4543 69.3243) (end 95.2843 71.1543) (width 0.508) (layer B.Cu) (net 7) (status 20))
 (segment (start 93.715 69.3243) (end 95.545 71.1543) (width 0.254) (layer B.Cu) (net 7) (status 20))
 (segment (start 95.545 71.1543) (end 96.035 71.1543) (width 0.508) (layer B.Cu) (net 7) (status 30))
 (segment (start 96.035 71.1543) (end 97.865 69.3243) (width 0.508) (layer B.Cu) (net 7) (status 30))
 (segment (start 95.2843 71.1543) (end 95.545 71.1543) (width 0.508) (layer B.Cu) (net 7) (status 30))
 (segment (start 98.445 64.8043) (end 98.445 65.893) (width 0.254) (layer F.Cu) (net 7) (status 10))
 (segment (start 98.445 65.893) (end 97.8154 66.5226) (width 0.254) (layer F.Cu) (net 7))
 (segment (start 97.8154 66.5226) (end 97.8154 69.2747) (width 0.254) (layer F.Cu) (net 7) (status 20))
 (segment (start 87.5957 66.675) (end 90.245 69.3243) (width 0.508) (layer B.Cu) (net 7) (status 20))
 (segment (start 90.245 69.3243) (end 93.4543 69.3243) (width 0.508) (layer B.Cu) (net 7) (status 10))
 (segment (start 90.245 69.3243) (end 93.715 69.3243) (width 0.254) (layer B.Cu) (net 7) (status 10))
 (segment (start 97.8154 69.2747) (end 97.865 69.3243) (width 0.254) (layer F.Cu) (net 7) (status 30))
 (segment (start 83.185 66.675) (end 87.5957 66.675) (width 0.508) (layer B.Cu) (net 7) (status 10))
 (segment (start 87.6357 69.215) (end 90.245 71.8243) (width 0.254) (layer B.Cu) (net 8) (status 20))
 (segment (start 95.545 71.9543) (end 90.375 71.9543) (width 0.254) (layer B.Cu) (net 8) (status 30))
 (segment (start 90.375 71.9543) (end 90.245 71.8243) (width 0.254) (layer B.Cu) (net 8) (status 30))
 (segment (start 96.7232 68.3514) (end 96.7232 70.6825) (width 0.254) (layer F.Cu) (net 8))
 (segment (start 96.7232 70.6825) (end 97.865 71.8243) (width 0.254) (layer F.Cu) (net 8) (status 20))
 (segment (start 97.735 71.9543) (end 97.865 71.8243) (width 0.254) (layer B.Cu) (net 8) (status 30))
 (segment (start 83.185 69.215) (end 87.6357 69.215) (width 0.254) (layer B.Cu) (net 8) (status 10))
 (segment (start 97.282 67.7926) (end 96.7232 68.3514) (width 0.254) (layer F.Cu) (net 8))
 (segment (start 97.282 66.3194) (end 97.282 67.7926) (width 0.254) (layer F.Cu) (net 8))
 (segment (start 97.795 65.8064) (end 97.282 66.3194) (width 0.254) (layer F.Cu) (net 8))
 (segment (start 97.795 64.8043) (end 97.795 65.8064) (width 0.254) (layer F.Cu) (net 8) (status 10))
 (segment (start 95.545 71.9543) (end 97.735 71.9543) (width 0.254) (layer B.Cu) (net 8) (status 30))
 (segment (start 88.1757 71.755) (end 90.245 73.8243) (width 0.254) (layer B.Cu) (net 9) (status 20))
 (segment (start 91.315 72.7543) (end 90.245 73.8243) (width 0.254) (layer B.Cu) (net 9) (status 20))
 (segment (start 96.1898 72.1491) (end 97.865 73.8243) (width 0.254) (layer F.Cu) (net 9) (status 20))
 (segment (start 83.185 71.755) (end 88.1757 71.755) (width 0.254) (layer B.Cu) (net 9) (status 10))
 (segment (start 96.1898 68.1482) (end 96.1898 72.1491) (width 0.254) (layer F.Cu) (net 9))
 (segment (start 96.7486 67.5894) (end 96.1898 68.1482) (width 0.254) (layer F.Cu) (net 9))
 (segment (start 96.7486 66.0908) (end 96.7486 67.5894) (width 0.254) (layer F.Cu) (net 9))
 (segment (start 97.145 65.6944) (end 96.7486 66.0908) (width 0.254) (layer F.Cu) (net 9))
 (segment (start 97.145 64.8043) (end 97.145 65.6944) (width 0.254) (layer F.Cu) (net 9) (status 10))
 (segment (start 96.795 72.7543) (end 97.865 73.8243) (width 0.254) (layer B.Cu) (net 9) (status 30))
 (segment (start 95.545 72.7543) (end 96.795 72.7543) (width 0.254) (layer B.Cu) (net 9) (status 30))
 (segment (start 95.545 72.7543) (end 91.315 72.7543) (width 0.254) (layer B.Cu) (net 9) (status 10))
 (segment (start 90.245 76.3243) (end 93.3477 76.3243) (width 0.508) (layer B.Cu) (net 11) (status 10))
 (segment (start 89.7343 76.835) (end 90.245 76.3243) (width 0.508) (layer B.Cu) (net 11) (status 30))
 (segment (start 95.6818 67.1322) (end 95.123 67.691) (width 0.254) (layer F.Cu) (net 11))
 (segment (start 95.845 64.8043) (end 95.845 65.4958) (width 0.254) (layer F.Cu) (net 11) (status 10))
 (segment (start 95.6818 65.659) (end 95.6818 67.1322) (width 0.254) (layer F.Cu) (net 11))
 (segment (start 95.845 65.4958) (end 95.6818 65.659) (width 0.254) (layer F.Cu) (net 11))
 (segment (start 95.123 67.691) (end 95.123 71.1962) (width 0.254) (layer F.Cu) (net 11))
 (segment (start 83.185 76.835) (end 89.7343 76.835) (width 0.508) (layer B.Cu) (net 11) (status 30))
 (segment (start 95.123 71.1962) (end 90.245 76.0742) (width 0.254) (layer F.Cu) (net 11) (status 20))
 (segment (start 90.245 76.0742) (end 90.245 76.3243) (width 0.254) (layer F.Cu) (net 11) (status 30))
 (segment (start 93.3477 76.3243) (end 95.3177 74.3543) (width 0.508) (layer B.Cu) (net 11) (status 20))
 (segment (start 95.545 74.3543) (end 95.895 74.3543) (width 0.508) (layer B.Cu) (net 11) (status 30))
 (segment (start 95.3177 74.3543) (end 95.545 74.3543) (width 0.508) (layer B.Cu) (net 11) (status 30))
 (segment (start 95.895 74.3543) (end 97.865 76.3243) (width 0.508) (layer B.Cu) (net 11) (status 30))
 (segment (start 100.445 64.6543) (end 100.445 66.4943) (width 0.508) (layer F.Cu) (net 12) (status 30))
 (segment (start 100.445 66.4943) (end 99.965 66.9743) (width 0.508) (layer F.Cu) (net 12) (status 30))
 (segment (start 99.97 62.4043) (end 99.97 64.1793) (width 0.508) (layer F.Cu) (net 12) (status 30))
 (segment (start 99.97 64.1793) (end 100.445 64.6543) (width 0.508) (layer F.Cu) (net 12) (status 30))
 (segment (start 93.845 64.6543) (end 93.845 65.3633) (width 0.508) (layer F.Cu) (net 12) (status 30))
 (segment (start 93.845 65.3633) (end 92.955 66.2533) (width 0.508) (layer F.Cu) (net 12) (status 30))
 (segment (start 94.32 62.4043) (end 94.32 64.1793) (width 0.508) (layer F.Cu) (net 12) (status 30))
 (segment (start 94.32 64.1793) (end 93.845 64.6543) (width 0.508) (layer F.Cu) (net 12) (status 30))
 (segment (start 92.955 79.3953) (end 83.2053 79.3953) (width 0.508) (layer B.Cu) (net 12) (status 30))
 (segment (start 83.2053 79.3953) (end 83.185 79.375) (width 0.508) (layer B.Cu) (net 12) (status 30))
 (segment (start 99.965 66.9743) (end 93.676 66.9743) (width 0.508) (layer B.Cu) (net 12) (status 30))
 (segment (start 93.676 66.9743) (end 92.955 66.2533) (width 0.508) (layer B.Cu) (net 12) (status 30))
 (segment (start 99.965 66.9743) (end 99.965 67.2743) (width 0.508) (layer B.Cu) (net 12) (status 30))
 (segment (start 99.965 67.2743) (end 101.045 68.3543) (width 0.508) (layer B.Cu) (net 12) (status 30))
 (segment (start 95.545 68.3543) (end 95.056 68.3543) (width 0.508) (layer B.Cu) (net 12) (status 30))
 (segment (start 95.056 68.3543) (end 92.955 66.2533) (width 0.508) (layer B.Cu) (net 12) (status 30))
 (segment (start 92.955 79.3953) (end 93.304 79.3953) (width 0.508) (layer B.Cu) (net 12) (status 30))
 (segment (start 93.304 79.3953) (end 95.545 77.1543) (width 0.508) (layer B.Cu) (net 12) (status 30))
 (segment (start 92.955 79.3953) (end 99.244 79.3953) (width 0.508) (layer B.Cu) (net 12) (status 30))
 (segment (start 99.244 79.3953) (end 99.965 78.6743) (width 0.508) (layer B.Cu) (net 12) (status 30))
 (segment (start 99.965 78.6743) (end 99.965 78.2343) (width 0.508) (layer B.Cu) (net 12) (status 30))
 (segment (start 99.965 78.2343) (end 101.045 77.1543) (width 0.508) (layer B.Cu) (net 12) (status 30))
 (segment (start 101.1 77.1) (end 101.05 77.15) (width 0.508) (layer B.Cu) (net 12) (status 30))
 (segment (start 101.05 70.05) (end 101.1 70.1) (width 0.508) (layer B.Cu) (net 12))
 (segment (start 101.1 70.1) (end 101.1 77.1) (width 0.508) (layer B.Cu) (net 12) (status 20))
 (segment (start 101.05 68.35) (end 101.05 70.05) (width 0.508) (layer B.Cu) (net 12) (status 10))
 (segment (start 83.947 75.057) (end 83.185 74.295) (width 0.254) (layer B.Cu) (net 10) (status 20))
 (segment (start 95.6564 71.8566) (end 93.599 73.914) (width 0.254) (layer F.Cu) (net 10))
 (segment (start 96.495 64.8043) (end 96.495 65.5824) (width 0.254) (layer F.Cu) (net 10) (status 10))
 (segment (start 96.2152 67.3608) (end 95.6564 67.9196) (width 0.254) (layer F.Cu) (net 10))
 (segment (start 96.2152 65.8622) (end 96.2152 67.3608) (width 0.254) (layer F.Cu) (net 10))
 (segment (start 96.495 65.5824) (end 96.2152 65.8622) (width 0.254) (layer F.Cu) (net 10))
 (segment (start 95.6564 67.9196) (end 95.6564 71.8566) (width 0.254) (layer F.Cu) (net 10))
 (via (at 93.599 73.914) (size 0.889) (layers F.Cu B.Cu) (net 10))
 (segment (start 90.678 75.057) (end 83.947 75.057) (width 0.254) (layer B.Cu) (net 10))
 (segment (start 91.821 73.914) (end 90.678 75.057) (width 0.254) (layer B.Cu) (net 10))
 (segment (start 95.545 73.5543) (end 93.9587 73.5543) (width 0.254) (layer B.Cu) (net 10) (status 10))
 (segment (start 93.9587 73.5543) (end 93.599 73.914) (width 0.254) (layer B.Cu) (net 10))
 (segment (start 93.599 73.914) (end 91.821 73.914) (width 0.254) (layer B.Cu) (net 10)))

